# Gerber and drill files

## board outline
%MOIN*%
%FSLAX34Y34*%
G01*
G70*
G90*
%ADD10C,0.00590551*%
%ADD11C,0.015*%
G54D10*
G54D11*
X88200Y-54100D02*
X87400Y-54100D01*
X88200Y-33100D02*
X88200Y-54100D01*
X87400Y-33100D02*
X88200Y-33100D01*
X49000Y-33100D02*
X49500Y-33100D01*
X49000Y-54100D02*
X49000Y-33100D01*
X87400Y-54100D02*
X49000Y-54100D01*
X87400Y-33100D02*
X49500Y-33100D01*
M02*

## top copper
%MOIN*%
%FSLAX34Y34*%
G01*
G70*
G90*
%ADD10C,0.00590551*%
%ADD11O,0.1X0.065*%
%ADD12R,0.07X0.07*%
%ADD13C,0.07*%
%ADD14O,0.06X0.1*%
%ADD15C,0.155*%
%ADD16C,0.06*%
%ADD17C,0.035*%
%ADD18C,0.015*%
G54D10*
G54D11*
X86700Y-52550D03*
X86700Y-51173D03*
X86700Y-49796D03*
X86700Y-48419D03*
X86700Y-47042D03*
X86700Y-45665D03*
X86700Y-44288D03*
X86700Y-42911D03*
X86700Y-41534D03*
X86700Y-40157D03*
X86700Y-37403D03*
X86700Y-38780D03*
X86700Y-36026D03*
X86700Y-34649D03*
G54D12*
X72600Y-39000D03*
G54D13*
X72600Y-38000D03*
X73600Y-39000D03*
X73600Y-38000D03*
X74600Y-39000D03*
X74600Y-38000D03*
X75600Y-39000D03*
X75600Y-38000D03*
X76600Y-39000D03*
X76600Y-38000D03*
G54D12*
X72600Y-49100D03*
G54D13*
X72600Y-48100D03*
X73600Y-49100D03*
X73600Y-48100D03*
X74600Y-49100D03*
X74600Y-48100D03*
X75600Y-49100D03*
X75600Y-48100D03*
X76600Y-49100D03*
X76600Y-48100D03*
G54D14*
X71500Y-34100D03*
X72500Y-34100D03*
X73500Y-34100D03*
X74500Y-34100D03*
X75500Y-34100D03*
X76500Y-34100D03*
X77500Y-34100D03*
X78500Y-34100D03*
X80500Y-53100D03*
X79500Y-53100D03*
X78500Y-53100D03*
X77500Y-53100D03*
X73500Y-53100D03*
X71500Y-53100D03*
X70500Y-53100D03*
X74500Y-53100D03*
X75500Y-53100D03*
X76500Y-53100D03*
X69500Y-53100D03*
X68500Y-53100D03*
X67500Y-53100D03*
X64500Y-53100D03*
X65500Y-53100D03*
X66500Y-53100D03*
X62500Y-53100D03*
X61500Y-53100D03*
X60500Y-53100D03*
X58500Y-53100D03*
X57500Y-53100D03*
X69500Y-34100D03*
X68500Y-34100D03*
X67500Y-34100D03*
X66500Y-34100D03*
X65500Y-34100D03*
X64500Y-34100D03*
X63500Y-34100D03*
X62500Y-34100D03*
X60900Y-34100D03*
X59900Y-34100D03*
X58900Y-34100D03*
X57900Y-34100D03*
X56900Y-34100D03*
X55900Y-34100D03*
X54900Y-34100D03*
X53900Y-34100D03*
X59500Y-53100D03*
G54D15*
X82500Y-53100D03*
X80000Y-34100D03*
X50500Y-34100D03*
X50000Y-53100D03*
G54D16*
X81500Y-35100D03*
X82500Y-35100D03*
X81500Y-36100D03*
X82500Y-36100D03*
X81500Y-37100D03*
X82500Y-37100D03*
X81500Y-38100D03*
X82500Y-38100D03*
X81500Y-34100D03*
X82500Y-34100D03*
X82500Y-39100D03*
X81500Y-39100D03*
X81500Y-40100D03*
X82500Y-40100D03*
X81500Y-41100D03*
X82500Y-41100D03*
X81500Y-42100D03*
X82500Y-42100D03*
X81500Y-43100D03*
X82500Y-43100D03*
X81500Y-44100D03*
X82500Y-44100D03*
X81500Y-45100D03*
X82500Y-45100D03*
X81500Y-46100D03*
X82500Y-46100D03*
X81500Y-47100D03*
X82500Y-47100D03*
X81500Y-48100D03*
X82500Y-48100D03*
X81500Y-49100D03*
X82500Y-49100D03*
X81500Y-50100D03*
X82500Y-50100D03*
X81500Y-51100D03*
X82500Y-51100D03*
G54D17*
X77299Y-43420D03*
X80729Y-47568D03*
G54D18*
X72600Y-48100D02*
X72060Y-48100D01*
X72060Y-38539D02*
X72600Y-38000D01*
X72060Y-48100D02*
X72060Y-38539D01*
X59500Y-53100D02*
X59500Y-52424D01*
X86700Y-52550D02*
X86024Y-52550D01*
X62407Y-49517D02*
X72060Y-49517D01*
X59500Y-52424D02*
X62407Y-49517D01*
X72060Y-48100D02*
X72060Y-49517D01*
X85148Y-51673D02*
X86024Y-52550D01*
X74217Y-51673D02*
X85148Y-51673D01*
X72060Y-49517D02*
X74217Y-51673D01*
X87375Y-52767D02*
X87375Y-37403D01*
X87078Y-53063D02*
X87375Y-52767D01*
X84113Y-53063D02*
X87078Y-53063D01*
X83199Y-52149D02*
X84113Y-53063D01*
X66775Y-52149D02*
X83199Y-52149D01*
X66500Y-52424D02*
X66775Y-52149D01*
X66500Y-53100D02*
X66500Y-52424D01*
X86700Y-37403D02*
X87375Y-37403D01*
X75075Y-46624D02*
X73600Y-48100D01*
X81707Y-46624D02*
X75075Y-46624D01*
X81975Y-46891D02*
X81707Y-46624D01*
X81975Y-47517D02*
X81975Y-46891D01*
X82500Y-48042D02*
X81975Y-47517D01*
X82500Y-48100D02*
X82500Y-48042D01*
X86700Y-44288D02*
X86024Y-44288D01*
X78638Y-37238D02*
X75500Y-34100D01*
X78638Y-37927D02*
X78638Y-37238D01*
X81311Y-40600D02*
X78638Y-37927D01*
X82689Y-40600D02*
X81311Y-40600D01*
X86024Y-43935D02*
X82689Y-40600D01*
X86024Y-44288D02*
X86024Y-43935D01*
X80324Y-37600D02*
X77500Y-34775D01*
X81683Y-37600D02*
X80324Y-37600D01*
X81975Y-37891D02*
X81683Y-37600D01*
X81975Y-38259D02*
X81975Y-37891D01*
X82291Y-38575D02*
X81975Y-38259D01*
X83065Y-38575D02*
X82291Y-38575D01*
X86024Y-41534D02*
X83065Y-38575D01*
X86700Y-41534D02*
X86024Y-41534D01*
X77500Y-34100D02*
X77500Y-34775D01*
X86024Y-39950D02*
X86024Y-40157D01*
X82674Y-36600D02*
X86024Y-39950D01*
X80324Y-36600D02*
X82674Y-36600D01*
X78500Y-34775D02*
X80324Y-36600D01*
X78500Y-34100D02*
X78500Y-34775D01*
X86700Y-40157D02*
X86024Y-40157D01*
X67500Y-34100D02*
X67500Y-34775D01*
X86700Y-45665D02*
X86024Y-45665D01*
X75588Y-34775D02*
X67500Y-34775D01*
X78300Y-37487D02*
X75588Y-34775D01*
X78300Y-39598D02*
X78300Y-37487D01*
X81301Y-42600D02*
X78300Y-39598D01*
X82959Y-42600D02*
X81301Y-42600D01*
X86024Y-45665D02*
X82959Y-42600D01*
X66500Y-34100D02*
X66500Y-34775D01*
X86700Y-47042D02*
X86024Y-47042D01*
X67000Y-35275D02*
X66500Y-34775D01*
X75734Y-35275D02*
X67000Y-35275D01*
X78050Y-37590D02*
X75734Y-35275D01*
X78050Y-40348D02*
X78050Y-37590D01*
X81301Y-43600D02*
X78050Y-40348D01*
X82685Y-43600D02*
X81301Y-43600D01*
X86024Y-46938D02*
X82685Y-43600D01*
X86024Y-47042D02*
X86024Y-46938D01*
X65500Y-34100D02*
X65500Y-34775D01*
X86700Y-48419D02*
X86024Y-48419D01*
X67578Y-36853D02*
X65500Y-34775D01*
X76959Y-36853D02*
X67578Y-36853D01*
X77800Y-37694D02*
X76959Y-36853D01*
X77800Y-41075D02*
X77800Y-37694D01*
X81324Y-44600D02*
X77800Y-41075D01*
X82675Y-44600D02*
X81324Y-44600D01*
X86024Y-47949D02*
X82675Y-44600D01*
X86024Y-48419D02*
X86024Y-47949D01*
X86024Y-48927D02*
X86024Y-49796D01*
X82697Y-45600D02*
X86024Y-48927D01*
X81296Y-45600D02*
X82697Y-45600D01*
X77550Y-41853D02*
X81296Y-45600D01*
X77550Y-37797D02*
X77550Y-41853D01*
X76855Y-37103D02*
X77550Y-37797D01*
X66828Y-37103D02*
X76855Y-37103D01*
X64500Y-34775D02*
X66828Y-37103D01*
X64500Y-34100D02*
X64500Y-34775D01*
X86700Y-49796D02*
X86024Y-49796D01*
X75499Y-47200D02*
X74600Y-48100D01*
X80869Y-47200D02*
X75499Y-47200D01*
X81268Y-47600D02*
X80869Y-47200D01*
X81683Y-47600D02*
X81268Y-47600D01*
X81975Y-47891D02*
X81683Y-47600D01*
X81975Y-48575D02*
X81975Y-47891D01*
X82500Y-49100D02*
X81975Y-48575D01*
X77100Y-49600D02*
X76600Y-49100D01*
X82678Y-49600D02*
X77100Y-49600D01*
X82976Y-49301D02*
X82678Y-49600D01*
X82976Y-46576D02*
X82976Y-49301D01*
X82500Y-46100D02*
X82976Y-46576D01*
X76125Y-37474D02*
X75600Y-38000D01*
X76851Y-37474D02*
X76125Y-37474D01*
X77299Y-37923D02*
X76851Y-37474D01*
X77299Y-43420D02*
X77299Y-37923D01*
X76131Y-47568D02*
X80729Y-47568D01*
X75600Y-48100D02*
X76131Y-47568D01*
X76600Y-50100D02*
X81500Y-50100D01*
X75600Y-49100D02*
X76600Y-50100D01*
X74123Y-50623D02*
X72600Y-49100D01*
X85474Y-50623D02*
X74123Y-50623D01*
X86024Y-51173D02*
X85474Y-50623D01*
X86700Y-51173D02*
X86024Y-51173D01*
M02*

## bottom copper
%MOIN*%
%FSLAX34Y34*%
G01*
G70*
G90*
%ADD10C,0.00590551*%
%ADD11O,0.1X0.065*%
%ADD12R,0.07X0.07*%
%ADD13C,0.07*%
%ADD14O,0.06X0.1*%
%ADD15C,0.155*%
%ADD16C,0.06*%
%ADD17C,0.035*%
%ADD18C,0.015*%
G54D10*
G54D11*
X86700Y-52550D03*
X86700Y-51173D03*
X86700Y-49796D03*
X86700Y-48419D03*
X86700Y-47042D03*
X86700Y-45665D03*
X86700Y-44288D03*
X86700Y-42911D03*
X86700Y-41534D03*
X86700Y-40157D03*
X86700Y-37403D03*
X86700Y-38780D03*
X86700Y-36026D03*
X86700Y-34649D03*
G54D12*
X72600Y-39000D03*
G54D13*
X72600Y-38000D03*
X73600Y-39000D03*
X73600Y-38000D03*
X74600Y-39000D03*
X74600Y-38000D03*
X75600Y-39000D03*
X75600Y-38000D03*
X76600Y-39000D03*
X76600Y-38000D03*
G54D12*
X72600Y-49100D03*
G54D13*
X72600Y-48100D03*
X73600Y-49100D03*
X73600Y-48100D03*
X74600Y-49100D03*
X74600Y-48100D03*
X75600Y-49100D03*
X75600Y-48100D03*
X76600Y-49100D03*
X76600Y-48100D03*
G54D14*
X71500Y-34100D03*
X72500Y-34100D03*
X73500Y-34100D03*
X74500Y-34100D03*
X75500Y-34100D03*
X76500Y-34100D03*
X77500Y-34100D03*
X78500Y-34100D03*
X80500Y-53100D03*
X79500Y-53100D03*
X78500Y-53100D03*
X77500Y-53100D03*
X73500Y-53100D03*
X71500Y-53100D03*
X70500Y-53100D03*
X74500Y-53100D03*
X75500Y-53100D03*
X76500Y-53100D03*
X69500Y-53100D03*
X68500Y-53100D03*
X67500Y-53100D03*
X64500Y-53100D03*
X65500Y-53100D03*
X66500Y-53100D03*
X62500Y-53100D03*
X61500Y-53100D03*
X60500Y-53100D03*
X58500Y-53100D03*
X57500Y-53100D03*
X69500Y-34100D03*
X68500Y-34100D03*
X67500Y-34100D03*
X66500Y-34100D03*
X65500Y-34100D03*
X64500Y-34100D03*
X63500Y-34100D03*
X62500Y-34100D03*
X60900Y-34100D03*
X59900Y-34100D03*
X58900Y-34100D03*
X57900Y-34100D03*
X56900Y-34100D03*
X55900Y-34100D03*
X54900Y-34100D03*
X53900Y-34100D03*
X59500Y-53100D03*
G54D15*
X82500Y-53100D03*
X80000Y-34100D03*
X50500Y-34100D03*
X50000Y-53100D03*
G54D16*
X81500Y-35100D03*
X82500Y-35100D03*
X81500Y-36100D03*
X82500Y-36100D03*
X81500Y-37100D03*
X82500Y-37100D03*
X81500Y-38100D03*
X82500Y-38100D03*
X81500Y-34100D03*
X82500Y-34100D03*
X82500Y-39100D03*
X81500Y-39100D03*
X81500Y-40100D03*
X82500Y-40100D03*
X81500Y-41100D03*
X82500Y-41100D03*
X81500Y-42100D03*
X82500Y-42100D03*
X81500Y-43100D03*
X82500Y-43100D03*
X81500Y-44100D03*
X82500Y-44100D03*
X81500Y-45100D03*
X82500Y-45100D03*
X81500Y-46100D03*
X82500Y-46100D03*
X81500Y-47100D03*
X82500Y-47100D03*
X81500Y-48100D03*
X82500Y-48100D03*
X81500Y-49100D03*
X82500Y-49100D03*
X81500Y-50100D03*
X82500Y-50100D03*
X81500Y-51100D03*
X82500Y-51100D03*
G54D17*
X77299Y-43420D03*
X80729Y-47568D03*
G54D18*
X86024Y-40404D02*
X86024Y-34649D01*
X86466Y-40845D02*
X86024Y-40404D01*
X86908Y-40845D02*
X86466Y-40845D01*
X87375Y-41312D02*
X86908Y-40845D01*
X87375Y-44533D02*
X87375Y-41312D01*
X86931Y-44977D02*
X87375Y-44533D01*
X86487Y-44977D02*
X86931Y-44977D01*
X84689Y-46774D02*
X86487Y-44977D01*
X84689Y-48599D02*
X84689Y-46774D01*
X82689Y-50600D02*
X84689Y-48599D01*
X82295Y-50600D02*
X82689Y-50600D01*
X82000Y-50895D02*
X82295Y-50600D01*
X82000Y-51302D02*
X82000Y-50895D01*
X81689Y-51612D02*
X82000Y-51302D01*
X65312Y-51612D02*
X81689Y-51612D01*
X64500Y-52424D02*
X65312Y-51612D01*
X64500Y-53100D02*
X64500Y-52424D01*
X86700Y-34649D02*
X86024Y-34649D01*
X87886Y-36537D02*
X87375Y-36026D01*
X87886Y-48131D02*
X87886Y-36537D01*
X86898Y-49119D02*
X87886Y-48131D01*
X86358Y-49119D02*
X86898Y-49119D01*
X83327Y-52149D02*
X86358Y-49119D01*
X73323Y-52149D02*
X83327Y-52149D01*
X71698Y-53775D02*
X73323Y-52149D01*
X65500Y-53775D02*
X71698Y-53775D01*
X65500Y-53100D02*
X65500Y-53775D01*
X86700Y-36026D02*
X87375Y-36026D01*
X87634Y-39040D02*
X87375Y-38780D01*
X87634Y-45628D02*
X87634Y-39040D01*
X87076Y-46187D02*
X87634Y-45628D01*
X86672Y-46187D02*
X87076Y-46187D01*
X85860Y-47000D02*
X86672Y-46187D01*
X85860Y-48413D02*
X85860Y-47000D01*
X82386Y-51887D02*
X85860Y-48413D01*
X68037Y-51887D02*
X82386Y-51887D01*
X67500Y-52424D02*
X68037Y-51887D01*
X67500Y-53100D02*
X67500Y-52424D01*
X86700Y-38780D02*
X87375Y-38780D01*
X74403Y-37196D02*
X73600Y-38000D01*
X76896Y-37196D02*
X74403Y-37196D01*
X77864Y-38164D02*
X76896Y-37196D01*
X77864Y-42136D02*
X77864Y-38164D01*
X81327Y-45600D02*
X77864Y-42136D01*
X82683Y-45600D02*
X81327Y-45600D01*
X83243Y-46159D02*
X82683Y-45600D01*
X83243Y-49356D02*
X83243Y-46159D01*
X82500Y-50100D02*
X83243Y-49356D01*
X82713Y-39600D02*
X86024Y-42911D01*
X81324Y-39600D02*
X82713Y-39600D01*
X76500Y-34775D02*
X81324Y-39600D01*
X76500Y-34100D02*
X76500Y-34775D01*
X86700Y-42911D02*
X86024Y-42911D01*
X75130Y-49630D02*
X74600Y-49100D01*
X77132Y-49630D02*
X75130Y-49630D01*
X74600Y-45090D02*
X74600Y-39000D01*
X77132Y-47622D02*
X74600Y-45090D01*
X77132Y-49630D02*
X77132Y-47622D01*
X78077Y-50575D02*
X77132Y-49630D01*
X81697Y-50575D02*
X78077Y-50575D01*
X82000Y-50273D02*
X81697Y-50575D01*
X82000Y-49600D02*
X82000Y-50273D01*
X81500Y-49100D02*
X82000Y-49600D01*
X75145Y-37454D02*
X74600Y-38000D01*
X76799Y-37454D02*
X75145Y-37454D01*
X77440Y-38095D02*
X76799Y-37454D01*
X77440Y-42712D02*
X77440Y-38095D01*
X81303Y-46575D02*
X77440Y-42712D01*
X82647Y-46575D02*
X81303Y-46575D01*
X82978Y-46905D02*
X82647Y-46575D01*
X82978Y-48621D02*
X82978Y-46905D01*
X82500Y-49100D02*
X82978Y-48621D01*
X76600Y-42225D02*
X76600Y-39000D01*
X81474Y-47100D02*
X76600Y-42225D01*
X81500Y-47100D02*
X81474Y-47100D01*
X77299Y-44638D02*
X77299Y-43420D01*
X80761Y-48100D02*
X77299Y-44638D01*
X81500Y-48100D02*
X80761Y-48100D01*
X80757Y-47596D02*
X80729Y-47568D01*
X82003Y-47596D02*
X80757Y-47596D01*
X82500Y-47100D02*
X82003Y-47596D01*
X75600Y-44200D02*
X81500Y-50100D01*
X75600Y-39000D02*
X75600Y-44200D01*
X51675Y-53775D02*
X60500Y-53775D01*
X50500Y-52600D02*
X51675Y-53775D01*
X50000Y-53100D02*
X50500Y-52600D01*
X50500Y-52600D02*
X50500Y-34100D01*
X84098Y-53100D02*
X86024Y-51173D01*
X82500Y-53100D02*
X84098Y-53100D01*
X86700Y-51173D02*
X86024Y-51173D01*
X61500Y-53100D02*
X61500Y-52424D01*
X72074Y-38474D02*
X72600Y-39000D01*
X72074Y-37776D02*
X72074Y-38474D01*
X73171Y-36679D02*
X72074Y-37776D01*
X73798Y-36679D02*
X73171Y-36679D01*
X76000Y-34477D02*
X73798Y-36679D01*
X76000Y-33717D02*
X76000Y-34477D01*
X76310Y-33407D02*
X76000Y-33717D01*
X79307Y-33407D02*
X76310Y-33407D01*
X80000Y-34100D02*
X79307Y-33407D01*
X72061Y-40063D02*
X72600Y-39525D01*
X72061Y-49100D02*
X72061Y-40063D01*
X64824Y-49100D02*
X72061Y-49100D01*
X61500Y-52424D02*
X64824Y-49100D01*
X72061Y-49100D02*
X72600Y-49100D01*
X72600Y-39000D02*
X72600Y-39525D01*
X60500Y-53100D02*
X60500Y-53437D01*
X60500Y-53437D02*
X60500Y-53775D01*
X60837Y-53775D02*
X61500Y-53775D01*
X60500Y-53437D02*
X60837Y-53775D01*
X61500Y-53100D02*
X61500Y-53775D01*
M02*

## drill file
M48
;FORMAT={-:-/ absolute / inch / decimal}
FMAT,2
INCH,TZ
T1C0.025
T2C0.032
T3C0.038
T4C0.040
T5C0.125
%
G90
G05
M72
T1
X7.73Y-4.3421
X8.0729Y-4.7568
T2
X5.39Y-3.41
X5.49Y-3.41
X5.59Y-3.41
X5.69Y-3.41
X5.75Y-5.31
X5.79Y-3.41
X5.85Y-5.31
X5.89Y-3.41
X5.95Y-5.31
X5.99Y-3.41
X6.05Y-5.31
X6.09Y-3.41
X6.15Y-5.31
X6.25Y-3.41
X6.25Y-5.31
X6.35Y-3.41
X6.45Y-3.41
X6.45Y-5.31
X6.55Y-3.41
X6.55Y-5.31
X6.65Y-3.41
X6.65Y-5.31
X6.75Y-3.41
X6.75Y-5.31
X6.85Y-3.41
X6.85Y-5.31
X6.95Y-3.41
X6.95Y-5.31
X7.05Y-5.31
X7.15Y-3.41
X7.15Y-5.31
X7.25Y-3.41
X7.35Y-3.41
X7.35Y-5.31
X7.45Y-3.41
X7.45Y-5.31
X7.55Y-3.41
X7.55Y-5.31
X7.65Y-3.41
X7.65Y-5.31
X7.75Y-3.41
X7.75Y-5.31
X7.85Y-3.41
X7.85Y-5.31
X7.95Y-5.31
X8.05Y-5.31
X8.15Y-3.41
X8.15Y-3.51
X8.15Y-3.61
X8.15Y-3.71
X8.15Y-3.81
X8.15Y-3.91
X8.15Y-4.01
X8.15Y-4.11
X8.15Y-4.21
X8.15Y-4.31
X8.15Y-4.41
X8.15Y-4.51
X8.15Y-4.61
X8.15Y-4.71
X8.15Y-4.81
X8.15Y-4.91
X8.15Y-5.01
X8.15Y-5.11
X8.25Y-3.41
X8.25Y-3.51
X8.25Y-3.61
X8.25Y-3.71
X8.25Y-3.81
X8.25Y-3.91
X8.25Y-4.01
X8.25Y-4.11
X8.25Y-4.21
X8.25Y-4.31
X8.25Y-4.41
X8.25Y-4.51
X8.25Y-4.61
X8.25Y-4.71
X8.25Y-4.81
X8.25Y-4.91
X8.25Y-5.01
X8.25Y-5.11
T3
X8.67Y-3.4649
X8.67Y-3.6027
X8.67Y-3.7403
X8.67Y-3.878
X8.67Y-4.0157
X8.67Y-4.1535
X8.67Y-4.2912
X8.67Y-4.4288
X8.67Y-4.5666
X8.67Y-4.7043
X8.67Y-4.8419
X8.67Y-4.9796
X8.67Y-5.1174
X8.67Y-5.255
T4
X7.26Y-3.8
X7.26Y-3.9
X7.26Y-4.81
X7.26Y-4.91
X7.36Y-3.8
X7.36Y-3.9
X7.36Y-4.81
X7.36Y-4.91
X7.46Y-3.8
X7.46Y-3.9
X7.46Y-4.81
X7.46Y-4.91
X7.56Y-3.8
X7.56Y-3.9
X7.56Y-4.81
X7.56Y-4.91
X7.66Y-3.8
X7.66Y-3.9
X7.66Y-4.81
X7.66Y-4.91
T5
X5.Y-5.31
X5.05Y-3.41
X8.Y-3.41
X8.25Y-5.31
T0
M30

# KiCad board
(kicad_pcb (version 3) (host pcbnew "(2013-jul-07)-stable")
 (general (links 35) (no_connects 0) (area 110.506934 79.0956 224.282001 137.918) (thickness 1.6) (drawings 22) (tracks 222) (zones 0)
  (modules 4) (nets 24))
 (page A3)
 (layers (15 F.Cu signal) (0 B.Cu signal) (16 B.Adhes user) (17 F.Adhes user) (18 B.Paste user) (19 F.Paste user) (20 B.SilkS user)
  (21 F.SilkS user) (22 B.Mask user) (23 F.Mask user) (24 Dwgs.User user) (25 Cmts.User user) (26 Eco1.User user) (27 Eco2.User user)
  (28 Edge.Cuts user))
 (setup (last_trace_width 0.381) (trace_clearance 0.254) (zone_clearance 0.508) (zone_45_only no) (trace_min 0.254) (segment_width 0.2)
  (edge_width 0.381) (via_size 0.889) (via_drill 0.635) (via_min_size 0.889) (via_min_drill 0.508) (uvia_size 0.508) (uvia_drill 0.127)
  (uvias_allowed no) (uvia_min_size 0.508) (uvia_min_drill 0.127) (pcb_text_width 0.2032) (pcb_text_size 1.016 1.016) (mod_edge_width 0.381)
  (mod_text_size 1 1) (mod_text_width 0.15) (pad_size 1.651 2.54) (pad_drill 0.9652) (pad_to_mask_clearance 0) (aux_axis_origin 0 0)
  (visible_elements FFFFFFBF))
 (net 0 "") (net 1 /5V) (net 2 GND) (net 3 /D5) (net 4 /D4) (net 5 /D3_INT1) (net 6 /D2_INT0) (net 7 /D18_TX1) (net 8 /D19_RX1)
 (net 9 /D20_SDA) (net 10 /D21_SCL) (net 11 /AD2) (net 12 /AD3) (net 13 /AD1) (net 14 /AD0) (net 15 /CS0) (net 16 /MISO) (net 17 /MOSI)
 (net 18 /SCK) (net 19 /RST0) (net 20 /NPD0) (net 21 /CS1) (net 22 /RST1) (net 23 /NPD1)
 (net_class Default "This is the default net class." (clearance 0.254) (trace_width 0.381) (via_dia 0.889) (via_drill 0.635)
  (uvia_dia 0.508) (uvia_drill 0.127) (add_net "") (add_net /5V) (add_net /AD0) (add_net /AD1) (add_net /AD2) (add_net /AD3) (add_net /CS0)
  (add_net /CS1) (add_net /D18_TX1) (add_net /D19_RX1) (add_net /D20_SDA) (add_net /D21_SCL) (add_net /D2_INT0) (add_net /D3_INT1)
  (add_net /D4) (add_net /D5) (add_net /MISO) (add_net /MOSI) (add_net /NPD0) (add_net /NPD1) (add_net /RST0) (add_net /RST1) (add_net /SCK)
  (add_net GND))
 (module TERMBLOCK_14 (layer F.Cu) (at 220.218 110.744 90)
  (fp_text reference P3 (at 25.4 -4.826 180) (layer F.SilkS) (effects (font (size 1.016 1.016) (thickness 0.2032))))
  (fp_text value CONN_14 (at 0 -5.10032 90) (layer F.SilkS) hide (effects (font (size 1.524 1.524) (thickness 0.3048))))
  (pad 1 thru_hole oval (at -22.73427 0 270) (size 1.651 2.54) (drill 0.9652) (layers *.Cu *.Mask F.SilkS) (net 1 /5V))
  (pad 2 thru_hole oval (at -19.23669 0 270) (size 1.651 2.54) (drill 0.9652) (layers *.Cu *.Mask F.SilkS) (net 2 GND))
  (pad 3 thru_hole oval (at -15.73911 0 270) (size 1.651 2.54) (drill 0.9652) (layers *.Cu *.Mask F.SilkS) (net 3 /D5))
  (pad 4 thru_hole oval (at -12.24153 0 270) (size 1.651 2.54) (drill 0.9652) (layers *.Cu *.Mask F.SilkS) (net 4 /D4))
  (pad 5 thru_hole oval (at -8.74395 0 270) (size 1.651 2.54) (drill 0.9652) (layers *.Cu *.Mask F.SilkS) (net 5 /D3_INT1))
  (pad 6 thru_hole oval (at -5.24637 0 270) (size 1.651 2.54) (drill 0.9652) (layers *.Cu *.Mask F.SilkS) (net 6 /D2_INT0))
  (pad 7 thru_hole oval (at -1.74879 0 270) (size 1.651 2.54) (drill 0.9652) (layers *.Cu *.Mask F.SilkS) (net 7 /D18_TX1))
  (pad 8 thru_hole oval (at 1.74879 0 90) (size 1.651 2.54) (drill 0.9652) (layers *.Cu *.Mask F.SilkS) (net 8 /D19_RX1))
  (pad 9 thru_hole oval (at 5.24637 0 90) (size 1.651 2.54) (drill 0.9652) (layers *.Cu *.Mask F.SilkS) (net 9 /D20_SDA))
  (pad 10 thru_hole oval (at 8.74395 0 90) (size 1.651 2.54) (drill 0.9652) (layers *.Cu *.Mask F.SilkS) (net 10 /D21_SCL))
  (pad 12 thru_hole oval (at 15.73911 0 90) (size 1.651 2.54) (drill 0.9652) (layers *.Cu *.Mask F.SilkS) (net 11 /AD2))
  (pad 11 thru_hole oval (at 12.24153 0 90) (size 1.651 2.54) (drill 0.9652) (layers *.Cu *.Mask F.SilkS) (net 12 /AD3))
  (pad 13 thru_hole oval (at 19.23669 0 270) (size 1.651 2.54) (drill 0.9652) (layers *.Cu *.Mask F.SilkS) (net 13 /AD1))
  (pad 14 thru_hole oval (at 22.73427 0 270) (size 1.651 2.54) (drill 0.9652) (layers *.Cu *.Mask F.SilkS) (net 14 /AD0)))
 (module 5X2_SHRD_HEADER (layer F.Cu) (at 189.484 97.79)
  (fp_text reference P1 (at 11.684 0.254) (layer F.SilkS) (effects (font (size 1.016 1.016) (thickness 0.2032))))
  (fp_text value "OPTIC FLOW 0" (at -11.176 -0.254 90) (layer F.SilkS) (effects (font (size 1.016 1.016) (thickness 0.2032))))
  (pad 1 thru_hole rect (at -5.08 1.27) (size 1.778 1.778) (drill 1.016) (layers *.Cu *.Mask F.SilkS) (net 2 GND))
  (pad 2 thru_hole circle (at -5.08 -1.27) (size 1.778 1.778) (drill 1.016) (layers *.Cu *.Mask F.SilkS) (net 1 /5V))
  (pad 3 thru_hole circle (at -2.54 1.27) (size 1.778 1.778) (drill 1.016) (layers *.Cu *.Mask F.SilkS))
  (pad 4 thru_hole circle (at -2.54 -1.27) (size 1.778 1.778) (drill 1.016) (layers *.Cu *.Mask F.SilkS) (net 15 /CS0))
  (pad 5 thru_hole circle (at 0 1.27) (size 1.778 1.778) (drill 1.016) (layers *.Cu *.Mask F.SilkS) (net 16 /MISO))
  (pad 6 thru_hole circle (at 0 -1.27) (size 1.778 1.778) (drill 1.016) (layers *.Cu *.Mask F.SilkS) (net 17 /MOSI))
  (pad 7 thru_hole circle (at 2.54 1.27) (size 1.778 1.778) (drill 1.016) (layers *.Cu *.Mask F.SilkS) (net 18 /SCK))
  (pad 8 thru_hole circle (at 2.54 -1.27) (size 1.778 1.778) (drill 1.016) (layers *.Cu *.Mask F.SilkS) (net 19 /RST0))
  (pad 9 thru_hole circle (at 5.08 1.27) (size 1.778 1.778) (drill 1.016) (layers *.Cu *.Mask F.SilkS) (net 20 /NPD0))
  (pad 10 thru_hole circle (at 5.08 -1.27) (size 1.778 1.778) (drill 1.016) (layers *.Cu *.Mask F.SilkS)))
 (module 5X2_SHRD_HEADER (layer F.Cu) (at 189.484 123.444)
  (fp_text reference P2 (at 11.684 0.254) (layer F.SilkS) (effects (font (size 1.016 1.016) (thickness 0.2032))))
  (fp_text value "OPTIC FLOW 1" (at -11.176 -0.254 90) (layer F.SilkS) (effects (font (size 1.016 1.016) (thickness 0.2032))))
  (pad 1 thru_hole rect (at -5.08 1.27) (size 1.778 1.778) (drill 1.016) (layers *.Cu *.Mask F.SilkS) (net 2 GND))
  (pad 2 thru_hole circle (at -5.08 -1.27) (size 1.778 1.778) (drill 1.016) (layers *.Cu *.Mask F.SilkS) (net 1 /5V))
  (pad 3 thru_hole circle (at -2.54 1.27) (size 1.778 1.778) (drill 1.016) (layers *.Cu *.Mask F.SilkS))
  (pad 4 thru_hole circle (at -2.54 -1.27) (size 1.778 1.778) (drill 1.016) (layers *.Cu *.Mask F.SilkS) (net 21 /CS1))
  (pad 5 thru_hole circle (at 0 1.27) (size 1.778 1.778) (drill 1.016) (layers *.Cu *.Mask F.SilkS) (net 16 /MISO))
  (pad 6 thru_hole circle (at 0 -1.27) (size 1.778 1.778) (drill 1.016) (layers *.Cu *.Mask F.SilkS) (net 17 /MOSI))
  (pad 7 thru_hole circle (at 2.54 1.27) (size 1.778 1.778) (drill 1.016) (layers *.Cu *.Mask F.SilkS) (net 18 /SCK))
  (pad 8 thru_hole circle (at 2.54 -1.27) (size 1.778 1.778) (drill 1.016) (layers *.Cu *.Mask F.SilkS) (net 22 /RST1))
  (pad 9 thru_hole circle (at 5.08 1.27) (size 1.778 1.778) (drill 1.016) (layers *.Cu *.Mask F.SilkS) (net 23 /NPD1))
  (pad 10 thru_hole circle (at 5.08 -1.27) (size 1.778 1.778) (drill 1.016) (layers *.Cu *.Mask F.SilkS)))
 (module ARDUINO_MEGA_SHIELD (layer F.Cu) (at 113.03 137.414)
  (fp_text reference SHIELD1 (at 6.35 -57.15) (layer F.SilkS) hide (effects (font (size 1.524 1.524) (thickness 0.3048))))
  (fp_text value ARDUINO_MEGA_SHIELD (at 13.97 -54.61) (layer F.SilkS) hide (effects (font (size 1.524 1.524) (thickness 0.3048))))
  (pad 14 thru_hole oval (at 68.58 -50.8 90) (size 2.54 1.524) (drill 0.8128) (layers *.Cu *.Mask F.SilkS))
  (pad 15 thru_hole oval (at 71.12 -50.8 90) (size 2.54 1.524) (drill 0.8128) (layers *.Cu *.Mask F.SilkS))
  (pad 16 thru_hole oval (at 73.66 -50.8 90) (size 2.54 1.524) (drill 0.8128) (layers *.Cu *.Mask F.SilkS))
  (pad 17 thru_hole oval (at 76.2 -50.8 90) (size 2.54 1.524) (drill 0.8128) (layers *.Cu *.Mask F.SilkS))
  (pad 18 thru_hole oval (at 78.74 -50.8 90) (size 2.54 1.524) (drill 0.8128) (layers *.Cu *.Mask F.SilkS) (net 7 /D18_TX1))
  (pad 19 thru_hole oval (at 81.28 -50.8 90) (size 2.54 1.524) (drill 0.8128) (layers *.Cu *.Mask F.SilkS) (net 8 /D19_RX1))
  (pad 20 thru_hole oval (at 83.82 -50.8 90) (size 2.54 1.524) (drill 0.8128) (layers *.Cu *.Mask F.SilkS) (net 9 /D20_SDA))
  (pad 21 thru_hole oval (at 86.36 -50.8 90) (size 2.54 1.524) (drill 0.8128) (layers *.Cu *.Mask F.SilkS) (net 10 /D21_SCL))
  (pad AD15 thru_hole oval (at 91.44 -2.54 90) (size 2.54 1.524) (drill 0.8128) (layers *.Cu *.Mask F.SilkS))
  (pad AD14 thru_hole oval (at 88.9 -2.54 90) (size 2.54 1.524) (drill 0.8128) (layers *.Cu *.Mask F.SilkS))
  (pad AD13 thru_hole oval (at 86.36 -2.54 90) (size 2.54 1.524) (drill 0.8128) (layers *.Cu *.Mask F.SilkS))
  (pad AD12 thru_hole oval (at 83.82 -2.54 90) (size 2.54 1.524) (drill 0.8128) (layers *.Cu *.Mask F.SilkS))
  (pad AD8 thru_hole oval (at 73.66 -2.54 90) (size 2.54 1.524) (drill 0.8128) (layers *.Cu *.Mask F.SilkS))
  (pad AD7 thru_hole oval (at 68.58 -2.54 90) (size 2.54 1.524) (drill 0.8128) (layers *.Cu *.Mask F.SilkS))
  (pad AD6 thru_hole oval (at 66.04 -2.54 90) (size 2.54 1.524) (drill 0.8128) (layers *.Cu *.Mask F.SilkS))
  (pad AD9 thru_hole oval (at 76.2 -2.54 90) (size 2.54 1.524) (drill 0.8128) (layers *.Cu *.Mask F.SilkS))
  (pad AD10 thru_hole oval (at 78.74 -2.54 90) (size 2.54 1.524) (drill 0.8128) (layers *.Cu *.Mask F.SilkS))
  (pad AD11 thru_hole oval (at 81.28 -2.54 90) (size 2.54 1.524) (drill 0.8128) (layers *.Cu *.Mask F.SilkS))
  (pad AD5 thru_hole oval (at 63.5 -2.54 90) (size 2.54 1.524) (drill 0.8128) (layers *.Cu *.Mask F.SilkS))
  (pad AD4 thru_hole oval (at 60.96 -2.54 90) (size 2.54 1.524) (drill 0.8128) (layers *.Cu *.Mask F.SilkS))
  (pad AD3 thru_hole oval (at 58.42 -2.54 90) (size 2.54 1.524) (drill 0.8128) (layers *.Cu *.Mask F.SilkS) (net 12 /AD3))
  (pad AD0 thru_hole oval (at 50.8 -2.54 90) (size 2.54 1.524) (drill 0.8128) (layers *.Cu *.Mask F.SilkS) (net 14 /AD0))
  (pad AD1 thru_hole oval (at 53.34 -2.54 90) (size 2.54 1.524) (drill 0.8128) (layers *.Cu *.Mask F.SilkS) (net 13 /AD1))
  (pad AD2 thru_hole oval (at 55.88 -2.54 90) (size 2.54 1.524) (drill 0.8128) (layers *.Cu *.Mask F.SilkS) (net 11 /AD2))
  (pad V_IN thru_hole oval (at 45.72 -2.54 90) (size 2.54 1.524) (drill 0.8128) (layers *.Cu *.Mask F.SilkS))
  (pad GND2 thru_hole oval (at 43.18 -2.54 90) (size 2.54 1.524) (drill 0.8128) (layers *.Cu *.Mask F.SilkS) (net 2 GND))
  (pad GND1 thru_hole oval (at 40.64 -2.54 90) (size 2.54 1.524) (drill 0.8128) (layers *.Cu *.Mask F.SilkS) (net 2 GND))
  (pad 3V3 thru_hole oval (at 35.56 -2.54 90) (size 2.54 1.524) (drill 0.8128) (layers *.Cu *.Mask F.SilkS))
  (pad RST thru_hole oval (at 33.02 -2.54 90) (size 2.54 1.524) (drill 0.8128) (layers *.Cu *.Mask F.SilkS))
  (pad 0 thru_hole oval (at 63.5 -50.8 90) (size 2.54 1.524) (drill 0.8128) (layers *.Cu *.Mask F.SilkS))
  (pad 1 thru_hole oval (at 60.96 -50.8 90) (size 2.54 1.524) (drill 0.8128) (layers *.Cu *.Mask F.SilkS))
  (pad 2 thru_hole oval (at 58.42 -50.8 90) (size 2.54 1.524) (drill 0.8128) (layers *.Cu *.Mask F.SilkS) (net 6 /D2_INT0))
  (pad 3 thru_hole oval (at 55.88 -50.8 90) (size 2.54 1.524) (drill 0.8128) (layers *.Cu *.Mask F.SilkS) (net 5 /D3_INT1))
  (pad 4 thru_hole oval (at 53.34 -50.8 90) (size 2.54 1.524) (drill 0.8128) (layers *.Cu *.Mask F.SilkS) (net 4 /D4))
  (pad 5 thru_hole oval (at 50.8 -50.8 90) (size 2.54 1.524) (drill 0.8128) (layers *.Cu *.Mask F.SilkS) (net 3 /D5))
  (pad 6 thru_hole oval (at 48.26 -50.8 90) (size 2.54 1.524) (drill 0.8128) (layers *.Cu *.Mask F.SilkS))
  (pad 7 thru_hole oval (at 45.72 -50.8 90) (size 2.54 1.524) (drill 0.8128) (layers *.Cu *.Mask F.SilkS))
  (pad 8 thru_hole oval (at 41.656 -50.8 90) (size 2.54 1.524) (drill 0.8128) (layers *.Cu *.Mask F.SilkS))
  (pad 9 thru_hole oval (at 39.116 -50.8 90) (size 2.54 1.524) (drill 0.8128) (layers *.Cu *.Mask F.SilkS))
  (pad 10 thru_hole oval (at 36.576 -50.8 90) (size 2.54 1.524) (drill 0.8128) (layers *.Cu *.Mask F.SilkS))
  (pad 11 thru_hole oval (at 34.036 -50.8 90) (size 2.54 1.524) (drill 0.8128) (layers *.Cu *.Mask F.SilkS))
  (pad 12 thru_hole oval (at 31.496 -50.8 90) (size 2.54 1.524) (drill 0.8128) (layers *.Cu *.Mask F.SilkS))
  (pad 13 thru_hole oval (at 28.956 -50.8 90) (size 2.54 1.524) (drill 0.8128) (layers *.Cu *.Mask F.SilkS))
  (pad GND3 thru_hole oval (at 26.416 -50.8 90) (size 2.54 1.524) (drill 0.8128) (layers *.Cu *.Mask F.SilkS))
  (pad AREF thru_hole oval (at 23.876 -50.8 90) (size 2.54 1.524) (drill 0.8128) (layers *.Cu *.Mask F.SilkS))
  (pad 5V thru_hole oval (at 38.1 -2.54 90) (size 2.54 1.524) (drill 0.8128) (layers *.Cu *.Mask F.SilkS) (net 1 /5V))
  (pad GND1 thru_hole circle (at 96.52 -2.54 90) (size 3.937 3.937) (drill 3.175) (layers *.Cu *.Mask F.SilkS) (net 2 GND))
  (pad GND1 thru_hole circle (at 90.17 -50.8 90) (size 3.937 3.937) (drill 3.175) (layers *.Cu *.Mask F.SilkS) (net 2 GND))
  (pad GND1 thru_hole circle (at 15.24 -50.8 90) (size 3.937 3.937) (drill 3.175) (layers *.Cu *.Mask F.SilkS) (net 2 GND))
  (pad GND1 thru_hole circle (at 13.97 -2.54 90) (size 3.937 3.937) (drill 3.175) (layers *.Cu *.Mask F.SilkS) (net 2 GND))
  (pad 22 thru_hole circle (at 93.98 -48.26) (size 1.524 1.524) (drill 0.8128) (layers *.Cu *.Mask F.SilkS))
  (pad 23 thru_hole circle (at 96.52 -48.26) (size 1.524 1.524) (drill 0.8128) (layers *.Cu *.Mask F.SilkS))
  (pad 24 thru_hole circle (at 93.98 -45.72) (size 1.524 1.524) (drill 0.8128) (layers *.Cu *.Mask F.SilkS))
  (pad 25 thru_hole circle (at 96.52 -45.72) (size 1.524 1.524) (drill 0.8128) (layers *.Cu *.Mask F.SilkS))
  (pad 26 thru_hole circle (at 93.98 -43.18) (size 1.524 1.524) (drill 0.8128) (layers *.Cu *.Mask F.SilkS))
  (pad 27 thru_hole circle (at 96.52 -43.18) (size 1.524 1.524) (drill 0.8128) (layers *.Cu *.Mask F.SilkS))
  (pad 28 thru_hole circle (at 93.98 -40.64) (size 1.524 1.524) (drill 0.8128) (layers *.Cu *.Mask F.SilkS))
  (pad 29 thru_hole circle (at 96.52 -40.64) (size 1.524 1.524) (drill 0.8128) (layers *.Cu *.Mask F.SilkS))
  (pad 5V_4 thru_hole circle (at 93.98 -50.8) (size 1.524 1.524) (drill 0.8128) (layers *.Cu *.Mask F.SilkS))
  (pad 5V_5 thru_hole circle (at 96.52 -50.8) (size 1.524 1.524) (drill 0.8128) (layers *.Cu *.Mask F.SilkS))
  (pad 31 thru_hole circle (at 96.52 -38.1) (size 1.524 1.524) (drill 0.8128) (layers *.Cu *.Mask F.SilkS))
  (pad 30 thru_hole circle (at 93.98 -38.1) (size 1.524 1.524) (drill 0.8128) (layers *.Cu *.Mask F.SilkS))
  (pad 32 thru_hole circle (at 93.98 -35.56) (size 1.524 1.524) (drill 0.8128) (layers *.Cu *.Mask F.SilkS))
  (pad 33 thru_hole circle (at 96.52 -35.56) (size 1.524 1.524) (drill 0.8128) (layers *.Cu *.Mask F.SilkS))
  (pad 34 thru_hole circle (at 93.98 -33.02) (size 1.524 1.524) (drill 0.8128) (layers *.Cu *.Mask F.SilkS))
  (pad 35 thru_hole circle (at 96.52 -33.02) (size 1.524 1.524) (drill 0.8128) (layers *.Cu *.Mask F.SilkS))
  (pad 36 thru_hole circle (at 93.98 -30.48) (size 1.524 1.524) (drill 0.8128) (layers *.Cu *.Mask F.SilkS))
  (pad 37 thru_hole circle (at 96.52 -30.48) (size 1.524 1.524) (drill 0.8128) (layers *.Cu *.Mask F.SilkS))
  (pad 38 thru_hole circle (at 93.98 -27.94) (size 1.524 1.524) (drill 0.8128) (layers *.Cu *.Mask F.SilkS))
  (pad 39 thru_hole circle (at 96.52 -27.94) (size 1.524 1.524) (drill 0.8128) (layers *.Cu *.Mask F.SilkS))
  (pad 40 thru_hole circle (at 93.98 -25.4) (size 1.524 1.524) (drill 0.8128) (layers *.Cu *.Mask F.SilkS))
  (pad 41 thru_hole circle (at 96.52 -25.4) (size 1.524 1.524) (drill 0.8128) (layers *.Cu *.Mask F.SilkS))
  (pad 42 thru_hole circle (at 93.98 -22.86) (size 1.524 1.524) (drill 0.8128) (layers *.Cu *.Mask F.SilkS))
  (pad 43 thru_hole circle (at 96.52 -22.86) (size 1.524 1.524) (drill 0.8128) (layers *.Cu *.Mask F.SilkS))
  (pad 44 thru_hole circle (at 93.98 -20.32) (size 1.524 1.524) (drill 0.8128) (layers *.Cu *.Mask F.SilkS))
  (pad 45 thru_hole circle (at 96.52 -20.32) (size 1.524 1.524) (drill 0.8128) (layers *.Cu *.Mask F.SilkS) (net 23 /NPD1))
  (pad 46 thru_hole circle (at 93.98 -17.78) (size 1.524 1.524) (drill 0.8128) (layers *.Cu *.Mask F.SilkS) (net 20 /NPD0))
  (pad 47 thru_hole circle (at 96.52 -17.78) (size 1.524 1.524) (drill 0.8128) (layers *.Cu *.Mask F.SilkS) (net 22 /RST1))
  (pad 48 thru_hole circle (at 93.98 -15.24) (size 1.524 1.524) (drill 0.8128) (layers *.Cu *.Mask F.SilkS) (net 19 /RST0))
  (pad 49 thru_hole circle (at 96.52 -15.24) (size 1.524 1.524) (drill 0.8128) (layers *.Cu *.Mask F.SilkS) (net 21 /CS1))
  (pad 50 thru_hole circle (at 93.98 -12.7) (size 1.524 1.524) (drill 0.8128) (layers *.Cu *.Mask F.SilkS) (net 16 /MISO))
  (pad 51 thru_hole circle (at 96.52 -12.7) (size 1.524 1.524) (drill 0.8128) (layers *.Cu *.Mask F.SilkS) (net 17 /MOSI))
  (pad 52 thru_hole circle (at 93.98 -10.16) (size 1.524 1.524) (drill 0.8128) (layers *.Cu *.Mask F.SilkS) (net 18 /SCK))
  (pad 53 thru_hole circle (at 96.52 -10.16) (size 1.524 1.524) (drill 0.8128) (layers *.Cu *.Mask F.SilkS) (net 15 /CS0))
  (pad GND4 thru_hole circle (at 93.98 -7.62) (size 1.524 1.524) (drill 0.8128) (layers *.Cu *.Mask F.SilkS))
  (pad GND5 thru_hole circle (at 96.52 -7.62) (size 1.524 1.524) (drill 0.8128) (layers *.Cu *.Mask F.SilkS)))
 (gr_line (start 224.028 137.414) (end 221.996 137.414) (angle 90) (layer Edge.Cuts) (width 0.381))
 (gr_line (start 224.028 84.074) (end 224.028 137.414) (angle 90) (layer Edge.Cuts) (width 0.381))
 (gr_line (start 221.996 84.074) (end 224.028 84.074) (angle 90) (layer Edge.Cuts) (width 0.381))
 (gr_line (start 124.46 84.074) (end 125.73 84.074) (angle 90) (layer Edge.Cuts) (width 0.381))
 (gr_line (start 124.46 137.414) (end 124.46 84.074) (angle 90) (layer Edge.Cuts) (width 0.381))
 (gr_line (start 221.996 137.414) (end 124.46 137.414) (angle 90) (layer Edge.Cuts) (width 0.381))
 (gr_line (start 221.996 84.074) (end 125.73 84.074) (angle 90) (layer Edge.Cuts) (width 0.381))
 (segment (start 184.404 122.174) (end 183.0347 122.174) (width 0.381) (layer F.Cu) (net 1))
 (segment (start 183.0347 97.8893) (end 184.404 96.52) (width 0.381) (layer F.Cu) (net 1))
 (segment (start 183.0347 122.174) (end 183.0347 97.8893) (width 0.381) (layer F.Cu) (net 1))
 (segment (start 151.13 134.874) (end 151.13 133.1592) (width 0.381) (layer F.Cu) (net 1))
 (segment (start 220.218 133.4783) (end 218.5032 133.4783) (width 0.381) (layer F.Cu) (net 1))
 (segment (start 158.5159 125.7733) (end 183.0347 125.7733) (width 0.381) (layer F.Cu) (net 1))
 (segment (start 151.13 133.1592) (end 158.5159 125.7733) (width 0.381) (layer F.Cu) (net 1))
 (segment (start 183.0347 122.174) (end 183.0347 125.7733) (width 0.381) (layer F.Cu) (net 1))
 (segment (start 216.276 131.2511) (end 218.5032 133.4783) (width 0.381) (layer F.Cu) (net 1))
 (segment (start 188.5125 131.2511) (end 216.276 131.2511) (width 0.381) (layer F.Cu) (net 1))
 (segment (start 183.0347 125.7733) (end 188.5125 131.2511) (width 0.381) (layer F.Cu) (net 1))
 (segment (start 218.5032 102.6271) (end 218.5032 88.0097) (width 0.381) (layer B.Cu) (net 14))
 (segment (start 219.6249 103.7488) (end 218.5032 102.6271) (width 0.381) (layer B.Cu) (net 14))
 (segment (start 220.7466 103.7488) (end 219.6249 103.7488) (width 0.381) (layer B.Cu) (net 14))
 (segment (start 221.9328 104.935) (end 220.7466 103.7488) (width 0.381) (layer B.Cu) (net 14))
 (segment (start 221.9328 113.1141) (end 221.9328 104.935) (width 0.381) (layer B.Cu) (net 14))
 (segment (start 220.8053 114.2416) (end 221.9328 113.1141) (width 0.381) (layer B.Cu) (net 14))
 (segment (start 219.6776 114.2416) (end 220.8053 114.2416) (width 0.381) (layer B.Cu) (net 14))
 (segment (start 215.1125 118.8067) (end 219.6776 114.2416) (width 0.381) (layer B.Cu) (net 14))
 (segment (start 215.1125 123.4433) (end 215.1125 118.8067) (width 0.381) (layer B.Cu) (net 14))
 (segment (start 210.0318 128.524) (end 215.1125 123.4433) (width 0.381) (layer B.Cu) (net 14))
 (segment (start 209.03 128.524) (end 210.0318 128.524) (width 0.381) (layer B.Cu) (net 14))
 (segment (start 208.28 129.274) (end 209.03 128.524) (width 0.381) (layer B.Cu) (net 14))
 (segment (start 208.28 130.3087) (end 208.28 129.274) (width 0.381) (layer B.Cu) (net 14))
 (segment (start 207.4925 131.0962) (end 208.28 130.3087) (width 0.381) (layer B.Cu) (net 14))
 (segment (start 165.893 131.0962) (end 207.4925 131.0962) (width 0.381) (layer B.Cu) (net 14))
 (segment (start 163.83 133.1592) (end 165.893 131.0962) (width 0.381) (layer B.Cu) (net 14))
 (segment (start 163.83 134.874) (end 163.83 133.1592) (width 0.381) (layer B.Cu) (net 14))
 (segment (start 220.218 88.0097) (end 218.5032 88.0097) (width 0.381) (layer B.Cu) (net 14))
 (segment (start 223.2318 92.8063) (end 221.9328 91.5073) (width 0.381) (layer B.Cu) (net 13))
 (segment (start 223.2318 122.2537) (end 223.2318 92.8063) (width 0.381) (layer B.Cu) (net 13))
 (segment (start 220.7222 124.7633) (end 223.2318 122.2537) (width 0.381) (layer B.Cu) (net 13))
 (segment (start 219.35 124.7633) (end 220.7222 124.7633) (width 0.381) (layer B.Cu) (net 13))
 (segment (start 211.6527 132.4606) (end 219.35 124.7633) (width 0.381) (layer B.Cu) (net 13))
 (segment (start 186.2427 132.4606) (end 211.6527 132.4606) (width 0.381) (layer B.Cu) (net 13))
 (segment (start 182.1145 136.5888) (end 186.2427 132.4606) (width 0.381) (layer B.Cu) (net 13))
 (segment (start 166.37 136.5888) (end 182.1145 136.5888) (width 0.381) (layer B.Cu) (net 13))
 (segment (start 166.37 134.874) (end 166.37 136.5888) (width 0.381) (layer B.Cu) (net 13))
 (segment (start 220.218 91.5073) (end 221.9328 91.5073) (width 0.381) (layer B.Cu) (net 13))
 (segment (start 221.9328 134.0294) (end 221.9328 95.0049) (width 0.381) (layer F.Cu) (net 11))
 (segment (start 221.1805 134.7817) (end 221.9328 134.0294) (width 0.381) (layer F.Cu) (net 11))
 (segment (start 213.6489 134.7817) (end 221.1805 134.7817) (width 0.381) (layer F.Cu) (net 11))
 (segment (start 211.3278 132.4606) (end 213.6489 134.7817) (width 0.381) (layer F.Cu) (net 11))
 (segment (start 169.6086 132.4606) (end 211.3278 132.4606) (width 0.381) (layer F.Cu) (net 11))
 (segment (start 168.91 133.1592) (end 169.6086 132.4606) (width 0.381) (layer F.Cu) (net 11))
 (segment (start 168.91 134.874) (end 168.91 133.1592) (width 0.381) (layer F.Cu) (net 11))
 (segment (start 220.218 95.0049) (end 221.9328 95.0049) (width 0.381) (layer F.Cu) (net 11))
 (segment (start 222.5924 99.1621) (end 221.9328 98.5025) (width 0.381) (layer B.Cu) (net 12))
 (segment (start 222.5924 115.8968) (end 222.5924 99.1621) (width 0.381) (layer B.Cu) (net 12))
 (segment (start 221.1737 117.3155) (end 222.5924 115.8968) (width 0.381) (layer B.Cu) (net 12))
 (segment (start 220.1491 117.3155) (end 221.1737 117.3155) (width 0.381) (layer B.Cu) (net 12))
 (segment (start 218.0844 119.3802) (end 220.1491 117.3155) (width 0.381) (layer B.Cu) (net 12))
 (segment (start 218.0844 122.9713) (end 218.0844 119.3802) (width 0.381) (layer B.Cu) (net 12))
 (segment (start 209.261 131.7947) (end 218.0844 122.9713) (width 0.381) (layer B.Cu) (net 12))
 (segment (start 172.8145 131.7947) (end 209.261 131.7947) (width 0.381) (layer B.Cu) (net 12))
 (segment (start 171.45 133.1592) (end 172.8145 131.7947) (width 0.381) (layer B.Cu) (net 12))
 (segment (start 171.45 134.874) (end 171.45 133.1592) (width 0.381) (layer B.Cu) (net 12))
 (segment (start 220.218 98.5025) (end 221.9328 98.5025) (width 0.381) (layer B.Cu) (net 12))
 (segment (start 188.9843 94.4797) (end 186.944 96.52) (width 0.381) (layer B.Cu) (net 15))
 (segment (start 195.3173 94.4797) (end 188.9843 94.4797) (width 0.381) (layer B.Cu) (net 15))
 (segment (start 197.7746 96.937) (end 195.3173 94.4797) (width 0.381) (layer B.Cu) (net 15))
 (segment (start 197.7746 107.026) (end 197.7746 96.937) (width 0.381) (layer B.Cu) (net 15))
 (segment (start 206.5726 115.824) (end 197.7746 107.026) (width 0.381) (layer B.Cu) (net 15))
 (segment (start 210.0169 115.824) (end 206.5726 115.824) (width 0.381) (layer B.Cu) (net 15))
 (segment (start 211.4379 117.245) (end 210.0169 115.824) (width 0.381) (layer B.Cu) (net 15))
 (segment (start 211.4379 125.3661) (end 211.4379 117.245) (width 0.381) (layer B.Cu) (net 15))
 (segment (start 209.55 127.254) (end 211.4379 125.3661) (width 0.381) (layer B.Cu) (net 15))
 (segment (start 190.6928 118.4252) (end 186.944 122.174) (width 0.381) (layer F.Cu) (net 21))
 (segment (start 207.5383 118.4252) (end 190.6928 118.4252) (width 0.381) (layer F.Cu) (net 21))
 (segment (start 208.2169 119.1038) (end 207.5383 118.4252) (width 0.381) (layer F.Cu) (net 21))
 (segment (start 208.2169 120.6942) (end 208.2169 119.1038) (width 0.381) (layer F.Cu) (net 21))
 (segment (start 209.55 122.0273) (end 208.2169 120.6942) (width 0.381) (layer F.Cu) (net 21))
 (segment (start 209.55 122.174) (end 209.55 122.0273) (width 0.381) (layer F.Cu) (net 21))
 (segment (start 220.218 112.4928) (end 218.5032 112.4928) (width 0.381) (layer F.Cu) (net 7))
 (segment (start 199.7427 94.5867) (end 191.77 86.614) (width 0.381) (layer F.Cu) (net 7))
 (segment (start 199.7427 96.3355) (end 199.7427 94.5867) (width 0.381) (layer F.Cu) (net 7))
 (segment (start 206.5312 103.124) (end 199.7427 96.3355) (width 0.381) (layer F.Cu) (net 7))
 (segment (start 210.0321 103.124) (end 206.5312 103.124) (width 0.381) (layer F.Cu) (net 7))
 (segment (start 218.5032 111.5951) (end 210.0321 103.124) (width 0.381) (layer F.Cu) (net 7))
 (segment (start 218.5032 112.4928) (end 218.5032 111.5951) (width 0.381) (layer F.Cu) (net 7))
 (segment (start 210.092 100.584) (end 218.5032 108.9952) (width 0.381) (layer B.Cu) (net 8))
 (segment (start 206.5652 100.584) (end 210.092 100.584) (width 0.381) (layer B.Cu) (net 8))
 (segment (start 194.31 88.3288) (end 206.5652 100.584) (width 0.381) (layer B.Cu) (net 8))
 (segment (start 194.31 86.614) (end 194.31 88.3288) (width 0.381) (layer B.Cu) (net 8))
 (segment (start 220.218 108.9952) (end 218.5032 108.9952) (width 0.381) (layer B.Cu) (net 8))
 (segment (start 204.0252 95.504) (end 196.85 88.3288) (width 0.381) (layer F.Cu) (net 9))
 (segment (start 207.4771 95.504) (end 204.0252 95.504) (width 0.381) (layer F.Cu) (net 9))
 (segment (start 208.2169 96.2438) (end 207.4771 95.504) (width 0.381) (layer F.Cu) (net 9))
 (segment (start 208.2169 97.1779) (end 208.2169 96.2438) (width 0.381) (layer F.Cu) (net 9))
 (segment (start 209.0199 97.9809) (end 208.2169 97.1779) (width 0.381) (layer F.Cu) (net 9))
 (segment (start 210.9865 97.9809) (end 209.0199 97.9809) (width 0.381) (layer F.Cu) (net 9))
 (segment (start 218.5032 105.4976) (end 210.9865 97.9809) (width 0.381) (layer F.Cu) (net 9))
 (segment (start 220.218 105.4976) (end 218.5032 105.4976) (width 0.381) (layer F.Cu) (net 9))
 (segment (start 196.85 86.614) (end 196.85 88.3288) (width 0.381) (layer F.Cu) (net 9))
 (segment (start 218.5032 101.4737) (end 218.5032 102) (width 0.381) (layer F.Cu) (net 10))
 (segment (start 209.9935 92.964) (end 218.5032 101.4737) (width 0.381) (layer F.Cu) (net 10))
 (segment (start 204.0252 92.964) (end 209.9935 92.964) (width 0.381) (layer F.Cu) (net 10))
 (segment (start 199.39 88.3288) (end 204.0252 92.964) (width 0.381) (layer F.Cu) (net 10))
 (segment (start 199.39 86.614) (end 199.39 88.3288) (width 0.381) (layer F.Cu) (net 10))
 (segment (start 220.218 102) (end 218.5032 102) (width 0.381) (layer F.Cu) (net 10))
 (segment (start 171.45 86.614) (end 171.45 88.3288) (width 0.381) (layer F.Cu) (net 6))
 (segment (start 220.218 115.9904) (end 218.5032 115.9904) (width 0.381) (layer F.Cu) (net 6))
 (segment (start 191.9942 88.3288) (end 171.45 88.3288) (width 0.381) (layer F.Cu) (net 6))
 (segment (start 198.8832 95.2178) (end 191.9942 88.3288) (width 0.381) (layer F.Cu) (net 6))
 (segment (start 198.8832 100.5802) (end 198.8832 95.2178) (width 0.381) (layer F.Cu) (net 6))
 (segment (start 206.507 108.204) (end 198.8832 100.5802) (width 0.381) (layer F.Cu) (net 6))
 (segment (start 210.7168 108.204) (end 206.507 108.204) (width 0.381) (layer F.Cu) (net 6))
 (segment (start 218.5032 115.9904) (end 210.7168 108.204) (width 0.381) (layer F.Cu) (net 6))
 (segment (start 168.91 86.614) (end 168.91 88.3288) (width 0.381) (layer F.Cu) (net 5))
 (segment (start 220.218 119.4879) (end 218.5032 119.4879) (width 0.381) (layer F.Cu) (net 5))
 (segment (start 170.1807 89.5995) (end 168.91 88.3288) (width 0.381) (layer F.Cu) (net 5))
 (segment (start 192.3665 89.5995) (end 170.1807 89.5995) (width 0.381) (layer F.Cu) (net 5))
 (segment (start 198.2476 95.4806) (end 192.3665 89.5995) (width 0.381) (layer F.Cu) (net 5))
 (segment (start 198.2476 102.4846) (end 198.2476 95.4806) (width 0.381) (layer F.Cu) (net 5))
 (segment (start 206.507 110.744) (end 198.2476 102.4846) (width 0.381) (layer F.Cu) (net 5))
 (segment (start 210.0224 110.744) (end 206.507 110.744) (width 0.381) (layer F.Cu) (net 5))
 (segment (start 218.5032 119.2248) (end 210.0224 110.744) (width 0.381) (layer F.Cu) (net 5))
 (segment (start 218.5032 119.4879) (end 218.5032 119.2248) (width 0.381) (layer F.Cu) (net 5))
 (segment (start 166.37 86.614) (end 166.37 88.3288) (width 0.381) (layer F.Cu) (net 4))
 (segment (start 220.218 122.9855) (end 218.5032 122.9855) (width 0.381) (layer F.Cu) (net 4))
 (segment (start 171.6496 93.6084) (end 166.37 88.3288) (width 0.381) (layer F.Cu) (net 4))
 (segment (start 195.477 93.6084) (end 171.6496 93.6084) (width 0.381) (layer F.Cu) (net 4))
 (segment (start 197.6123 95.7437) (end 195.477 93.6084) (width 0.381) (layer F.Cu) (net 4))
 (segment (start 197.6123 104.3328) (end 197.6123 95.7437) (width 0.381) (layer F.Cu) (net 4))
 (segment (start 206.5635 113.284) (end 197.6123 104.3328) (width 0.381) (layer F.Cu) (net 4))
 (segment (start 209.9965 113.284) (end 206.5635 113.284) (width 0.381) (layer F.Cu) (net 4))
 (segment (start 218.5032 121.7907) (end 209.9965 113.284) (width 0.381) (layer F.Cu) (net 4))
 (segment (start 218.5032 122.9855) (end 218.5032 121.7907) (width 0.381) (layer F.Cu) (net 4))
 (segment (start 218.5032 124.2756) (end 218.5032 126.4831) (width 0.381) (layer F.Cu) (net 3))
 (segment (start 210.0516 115.824) (end 218.5032 124.2756) (width 0.381) (layer F.Cu) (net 3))
 (segment (start 206.4933 115.824) (end 210.0516 115.824) (width 0.381) (layer F.Cu) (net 3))
 (segment (start 196.977 106.3077) (end 206.4933 115.824) (width 0.381) (layer F.Cu) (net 3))
 (segment (start 196.977 96.0068) (end 196.977 106.3077) (width 0.381) (layer F.Cu) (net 3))
 (segment (start 195.2139 94.2437) (end 196.977 96.0068) (width 0.381) (layer F.Cu) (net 3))
 (segment (start 169.7449 94.2437) (end 195.2139 94.2437) (width 0.381) (layer F.Cu) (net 3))
 (segment (start 163.83 88.3288) (end 169.7449 94.2437) (width 0.381) (layer F.Cu) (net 3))
 (segment (start 163.83 86.614) (end 163.83 88.3288) (width 0.381) (layer F.Cu) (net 3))
 (segment (start 220.218 126.4831) (end 218.5032 126.4831) (width 0.381) (layer F.Cu) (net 3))
 (segment (start 190.8309 126.0609) (end 189.484 124.714) (width 0.381) (layer B.Cu) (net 16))
 (segment (start 195.9164 126.0609) (end 190.8309 126.0609) (width 0.381) (layer B.Cu) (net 16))
 (segment (start 189.484 114.529) (end 189.484 99.06) (width 0.381) (layer B.Cu) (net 16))
 (segment (start 195.9164 120.9614) (end 189.484 114.529) (width 0.381) (layer B.Cu) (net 16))
 (segment (start 195.9164 126.0609) (end 195.9164 120.9614) (width 0.381) (layer B.Cu) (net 16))
 (segment (start 198.3174 128.4619) (end 195.9164 126.0609) (width 0.381) (layer B.Cu) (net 16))
 (segment (start 207.5125 128.4619) (end 198.3174 128.4619) (width 0.381) (layer B.Cu) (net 16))
 (segment (start 208.2801 127.6943) (end 207.5125 128.4619) (width 0.381) (layer B.Cu) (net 16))
 (segment (start 208.2801 125.9841) (end 208.2801 127.6943) (width 0.381) (layer B.Cu) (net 16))
 (segment (start 207.01 124.714) (end 208.2801 125.9841) (width 0.381) (layer B.Cu) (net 16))
 (segment (start 191.7676 119.8904) (end 189.484 122.174) (width 0.381) (layer F.Cu) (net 17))
 (segment (start 205.4082 119.8904) (end 191.7676 119.8904) (width 0.381) (layer F.Cu) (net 17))
 (segment (start 206.4218 120.904) (end 205.4082 119.8904) (width 0.381) (layer F.Cu) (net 17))
 (segment (start 207.4771 120.904) (end 206.4218 120.904) (width 0.381) (layer F.Cu) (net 17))
 (segment (start 208.2169 121.6438) (end 207.4771 120.904) (width 0.381) (layer F.Cu) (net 17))
 (segment (start 208.2169 123.3809) (end 208.2169 121.6438) (width 0.381) (layer F.Cu) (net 17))
 (segment (start 209.55 124.714) (end 208.2169 123.3809) (width 0.381) (layer F.Cu) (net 17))
 (segment (start 190.8708 95.1332) (end 189.484 96.52) (width 0.381) (layer B.Cu) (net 17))
 (segment (start 195.0699 95.1332) (end 190.8708 95.1332) (width 0.381) (layer B.Cu) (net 17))
 (segment (start 196.6993 96.7626) (end 195.0699 95.1332) (width 0.381) (layer B.Cu) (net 17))
 (segment (start 196.6993 108.4899) (end 196.6993 96.7626) (width 0.381) (layer B.Cu) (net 17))
 (segment (start 206.5102 118.3008) (end 196.6993 108.4899) (width 0.381) (layer B.Cu) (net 17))
 (segment (start 209.9259 118.3008) (end 206.5102 118.3008) (width 0.381) (layer B.Cu) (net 17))
 (segment (start 210.7642 119.1391) (end 209.9259 118.3008) (width 0.381) (layer B.Cu) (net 17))
 (segment (start 210.7642 123.4998) (end 210.7642 119.1391) (width 0.381) (layer B.Cu) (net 17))
 (segment (start 209.55 124.714) (end 210.7642 123.4998) (width 0.381) (layer B.Cu) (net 17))
 (segment (start 194.564 107.2532) (end 194.564 99.06) (width 0.381) (layer B.Cu) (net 20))
 (segment (start 206.9448 119.634) (end 194.564 107.2532) (width 0.381) (layer B.Cu) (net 20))
 (segment (start 207.01 119.634) (end 206.9448 119.634) (width 0.381) (layer B.Cu) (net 20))
 (segment (start 195.834 125.984) (end 194.564 124.714) (width 0.381) (layer F.Cu) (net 23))
 (segment (start 210.0025 125.984) (end 195.834 125.984) (width 0.381) (layer F.Cu) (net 23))
 (segment (start 210.7598 125.2267) (end 210.0025 125.984) (width 0.381) (layer F.Cu) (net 23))
 (segment (start 210.7598 118.3038) (end 210.7598 125.2267) (width 0.381) (layer F.Cu) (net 23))
 (segment (start 209.55 117.094) (end 210.7598 118.3038) (width 0.381) (layer F.Cu) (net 23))
 (via (at 196.3416 110.2889) (size 0.889) (layers F.Cu B.Cu) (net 19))
 (segment (start 196.3416 113.3819) (end 196.3416 110.2889) (width 0.381) (layer B.Cu) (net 19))
 (segment (start 205.1337 122.174) (end 196.3416 113.3819) (width 0.381) (layer B.Cu) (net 19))
 (segment (start 207.01 122.174) (end 205.1337 122.174) (width 0.381) (layer B.Cu) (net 19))
 (segment (start 193.3578 95.1862) (end 192.024 96.52) (width 0.381) (layer F.Cu) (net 19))
 (segment (start 195.2024 95.1862) (end 193.3578 95.1862) (width 0.381) (layer F.Cu) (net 19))
 (segment (start 196.3416 96.3254) (end 195.2024 95.1862) (width 0.381) (layer F.Cu) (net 19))
 (segment (start 196.3416 110.2889) (end 196.3416 96.3254) (width 0.381) (layer F.Cu) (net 19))
 (via (at 205.0524 120.8235) (size 0.889) (layers F.Cu B.Cu) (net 22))
 (segment (start 205.1242 120.8953) (end 205.0524 120.8235) (width 0.381) (layer B.Cu) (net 22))
 (segment (start 208.2887 120.8953) (end 205.1242 120.8953) (width 0.381) (layer B.Cu) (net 22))
 (segment (start 209.55 119.634) (end 208.2887 120.8953) (width 0.381) (layer B.Cu) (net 22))
 (segment (start 193.3745 120.8235) (end 205.0524 120.8235) (width 0.381) (layer F.Cu) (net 22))
 (segment (start 192.024 122.174) (end 193.3745 120.8235) (width 0.381) (layer F.Cu) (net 22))
 (segment (start 194.564 127.254) (end 207.01 127.254) (width 0.381) (layer F.Cu) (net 18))
 (segment (start 192.024 124.714) (end 194.564 127.254) (width 0.381) (layer F.Cu) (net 18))
 (segment (start 192.024 112.268) (end 207.01 127.254) (width 0.381) (layer B.Cu) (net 18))
 (segment (start 192.024 99.06) (end 192.024 112.268) (width 0.381) (layer B.Cu) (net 18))
 (segment (start 131.2548 136.5888) (end 153.67 136.5888) (width 0.381) (layer B.Cu) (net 2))
 (segment (start 128.27 133.604) (end 131.2548 136.5888) (width 0.381) (layer B.Cu) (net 2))
 (segment (start 127 134.874) (end 128.27 133.604) (width 0.381) (layer B.Cu) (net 2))
 (segment (start 128.27 133.604) (end 128.27 86.614) (width 0.381) (layer B.Cu) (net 2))
 (segment (start 213.6099 134.874) (end 218.5032 129.9807) (width 0.381) (layer B.Cu) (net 2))
 (segment (start 209.55 134.874) (end 213.6099 134.874) (width 0.381) (layer B.Cu) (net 2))
 (segment (start 220.218 129.9807) (end 218.5032 129.9807) (width 0.381) (layer B.Cu) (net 2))
 (segment (start 156.21 134.874) (end 156.21 133.1592) (width 0.381) (layer B.Cu) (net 2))
 (segment (start 183.0701 97.7261) (end 184.404 99.06) (width 0.381) (layer B.Cu) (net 2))
 (segment (start 183.0701 95.952) (end 183.0701 97.7261) (width 0.381) (layer B.Cu) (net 2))
 (segment (start 185.8562 93.1659) (end 183.0701 95.952) (width 0.381) (layer B.Cu) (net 2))
 (segment (start 187.4476 93.1659) (end 185.8562 93.1659) (width 0.381) (layer B.Cu) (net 2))
 (segment (start 193.04 87.5735) (end 187.4476 93.1659) (width 0.381) (layer B.Cu) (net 2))
 (segment (start 193.04 85.643) (end 193.04 87.5735) (width 0.381) (layer B.Cu) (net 2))
 (segment (start 193.8283 84.8547) (end 193.04 85.643) (width 0.381) (layer B.Cu) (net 2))
 (segment (start 201.4407 84.8547) (end 193.8283 84.8547) (width 0.381) (layer B.Cu) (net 2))
 (segment (start 203.2 86.614) (end 201.4407 84.8547) (width 0.381) (layer B.Cu) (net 2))
 (segment (start 188.2736 128.5836) (end 184.404 124.714) (width 0.381) (layer F.Cu) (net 2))
 (segment (start 217.1061 128.5836) (end 188.2736 128.5836) (width 0.381) (layer F.Cu) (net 2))
 (segment (start 218.5032 129.9807) (end 217.1061 128.5836) (width 0.381) (layer F.Cu) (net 2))
 (segment (start 220.218 129.9807) (end 218.5032 129.9807) (width 0.381) (layer F.Cu) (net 2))
 (segment (start 183.0356 101.7622) (end 184.404 100.3938) (width 0.381) (layer B.Cu) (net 2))
 (segment (start 183.0356 124.714) (end 183.0356 101.7622) (width 0.381) (layer B.Cu) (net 2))
 (segment (start 164.6552 124.714) (end 183.0356 124.714) (width 0.381) (layer B.Cu) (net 2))
 (segment (start 156.21 133.1592) (end 164.6552 124.714) (width 0.381) (layer B.Cu) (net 2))
 (segment (start 183.0356 124.714) (end 184.404 124.714) (width 0.381) (layer B.Cu) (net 2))
 (segment (start 184.404 99.06) (end 184.404 100.3938) (width 0.381) (layer B.Cu) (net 2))
 (segment (start 153.67 134.874) (end 153.67 135.7314) (width 0.381) (layer B.Cu) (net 2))
 (segment (start 153.67 135.7314) (end 153.67 136.5888) (width 0.381) (layer B.Cu) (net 2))
 (segment (start 154.5274 136.5888) (end 156.21 136.5888) (width 0.381) (layer B.Cu) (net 2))
 (segment (start 153.67 135.7314) (end 154.5274 136.5888) (width 0.381) (layer B.Cu) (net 2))
 (segment (start 156.21 134.874) (end 156.21 136.5888) (width 0.381) (layer B.Cu) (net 2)))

